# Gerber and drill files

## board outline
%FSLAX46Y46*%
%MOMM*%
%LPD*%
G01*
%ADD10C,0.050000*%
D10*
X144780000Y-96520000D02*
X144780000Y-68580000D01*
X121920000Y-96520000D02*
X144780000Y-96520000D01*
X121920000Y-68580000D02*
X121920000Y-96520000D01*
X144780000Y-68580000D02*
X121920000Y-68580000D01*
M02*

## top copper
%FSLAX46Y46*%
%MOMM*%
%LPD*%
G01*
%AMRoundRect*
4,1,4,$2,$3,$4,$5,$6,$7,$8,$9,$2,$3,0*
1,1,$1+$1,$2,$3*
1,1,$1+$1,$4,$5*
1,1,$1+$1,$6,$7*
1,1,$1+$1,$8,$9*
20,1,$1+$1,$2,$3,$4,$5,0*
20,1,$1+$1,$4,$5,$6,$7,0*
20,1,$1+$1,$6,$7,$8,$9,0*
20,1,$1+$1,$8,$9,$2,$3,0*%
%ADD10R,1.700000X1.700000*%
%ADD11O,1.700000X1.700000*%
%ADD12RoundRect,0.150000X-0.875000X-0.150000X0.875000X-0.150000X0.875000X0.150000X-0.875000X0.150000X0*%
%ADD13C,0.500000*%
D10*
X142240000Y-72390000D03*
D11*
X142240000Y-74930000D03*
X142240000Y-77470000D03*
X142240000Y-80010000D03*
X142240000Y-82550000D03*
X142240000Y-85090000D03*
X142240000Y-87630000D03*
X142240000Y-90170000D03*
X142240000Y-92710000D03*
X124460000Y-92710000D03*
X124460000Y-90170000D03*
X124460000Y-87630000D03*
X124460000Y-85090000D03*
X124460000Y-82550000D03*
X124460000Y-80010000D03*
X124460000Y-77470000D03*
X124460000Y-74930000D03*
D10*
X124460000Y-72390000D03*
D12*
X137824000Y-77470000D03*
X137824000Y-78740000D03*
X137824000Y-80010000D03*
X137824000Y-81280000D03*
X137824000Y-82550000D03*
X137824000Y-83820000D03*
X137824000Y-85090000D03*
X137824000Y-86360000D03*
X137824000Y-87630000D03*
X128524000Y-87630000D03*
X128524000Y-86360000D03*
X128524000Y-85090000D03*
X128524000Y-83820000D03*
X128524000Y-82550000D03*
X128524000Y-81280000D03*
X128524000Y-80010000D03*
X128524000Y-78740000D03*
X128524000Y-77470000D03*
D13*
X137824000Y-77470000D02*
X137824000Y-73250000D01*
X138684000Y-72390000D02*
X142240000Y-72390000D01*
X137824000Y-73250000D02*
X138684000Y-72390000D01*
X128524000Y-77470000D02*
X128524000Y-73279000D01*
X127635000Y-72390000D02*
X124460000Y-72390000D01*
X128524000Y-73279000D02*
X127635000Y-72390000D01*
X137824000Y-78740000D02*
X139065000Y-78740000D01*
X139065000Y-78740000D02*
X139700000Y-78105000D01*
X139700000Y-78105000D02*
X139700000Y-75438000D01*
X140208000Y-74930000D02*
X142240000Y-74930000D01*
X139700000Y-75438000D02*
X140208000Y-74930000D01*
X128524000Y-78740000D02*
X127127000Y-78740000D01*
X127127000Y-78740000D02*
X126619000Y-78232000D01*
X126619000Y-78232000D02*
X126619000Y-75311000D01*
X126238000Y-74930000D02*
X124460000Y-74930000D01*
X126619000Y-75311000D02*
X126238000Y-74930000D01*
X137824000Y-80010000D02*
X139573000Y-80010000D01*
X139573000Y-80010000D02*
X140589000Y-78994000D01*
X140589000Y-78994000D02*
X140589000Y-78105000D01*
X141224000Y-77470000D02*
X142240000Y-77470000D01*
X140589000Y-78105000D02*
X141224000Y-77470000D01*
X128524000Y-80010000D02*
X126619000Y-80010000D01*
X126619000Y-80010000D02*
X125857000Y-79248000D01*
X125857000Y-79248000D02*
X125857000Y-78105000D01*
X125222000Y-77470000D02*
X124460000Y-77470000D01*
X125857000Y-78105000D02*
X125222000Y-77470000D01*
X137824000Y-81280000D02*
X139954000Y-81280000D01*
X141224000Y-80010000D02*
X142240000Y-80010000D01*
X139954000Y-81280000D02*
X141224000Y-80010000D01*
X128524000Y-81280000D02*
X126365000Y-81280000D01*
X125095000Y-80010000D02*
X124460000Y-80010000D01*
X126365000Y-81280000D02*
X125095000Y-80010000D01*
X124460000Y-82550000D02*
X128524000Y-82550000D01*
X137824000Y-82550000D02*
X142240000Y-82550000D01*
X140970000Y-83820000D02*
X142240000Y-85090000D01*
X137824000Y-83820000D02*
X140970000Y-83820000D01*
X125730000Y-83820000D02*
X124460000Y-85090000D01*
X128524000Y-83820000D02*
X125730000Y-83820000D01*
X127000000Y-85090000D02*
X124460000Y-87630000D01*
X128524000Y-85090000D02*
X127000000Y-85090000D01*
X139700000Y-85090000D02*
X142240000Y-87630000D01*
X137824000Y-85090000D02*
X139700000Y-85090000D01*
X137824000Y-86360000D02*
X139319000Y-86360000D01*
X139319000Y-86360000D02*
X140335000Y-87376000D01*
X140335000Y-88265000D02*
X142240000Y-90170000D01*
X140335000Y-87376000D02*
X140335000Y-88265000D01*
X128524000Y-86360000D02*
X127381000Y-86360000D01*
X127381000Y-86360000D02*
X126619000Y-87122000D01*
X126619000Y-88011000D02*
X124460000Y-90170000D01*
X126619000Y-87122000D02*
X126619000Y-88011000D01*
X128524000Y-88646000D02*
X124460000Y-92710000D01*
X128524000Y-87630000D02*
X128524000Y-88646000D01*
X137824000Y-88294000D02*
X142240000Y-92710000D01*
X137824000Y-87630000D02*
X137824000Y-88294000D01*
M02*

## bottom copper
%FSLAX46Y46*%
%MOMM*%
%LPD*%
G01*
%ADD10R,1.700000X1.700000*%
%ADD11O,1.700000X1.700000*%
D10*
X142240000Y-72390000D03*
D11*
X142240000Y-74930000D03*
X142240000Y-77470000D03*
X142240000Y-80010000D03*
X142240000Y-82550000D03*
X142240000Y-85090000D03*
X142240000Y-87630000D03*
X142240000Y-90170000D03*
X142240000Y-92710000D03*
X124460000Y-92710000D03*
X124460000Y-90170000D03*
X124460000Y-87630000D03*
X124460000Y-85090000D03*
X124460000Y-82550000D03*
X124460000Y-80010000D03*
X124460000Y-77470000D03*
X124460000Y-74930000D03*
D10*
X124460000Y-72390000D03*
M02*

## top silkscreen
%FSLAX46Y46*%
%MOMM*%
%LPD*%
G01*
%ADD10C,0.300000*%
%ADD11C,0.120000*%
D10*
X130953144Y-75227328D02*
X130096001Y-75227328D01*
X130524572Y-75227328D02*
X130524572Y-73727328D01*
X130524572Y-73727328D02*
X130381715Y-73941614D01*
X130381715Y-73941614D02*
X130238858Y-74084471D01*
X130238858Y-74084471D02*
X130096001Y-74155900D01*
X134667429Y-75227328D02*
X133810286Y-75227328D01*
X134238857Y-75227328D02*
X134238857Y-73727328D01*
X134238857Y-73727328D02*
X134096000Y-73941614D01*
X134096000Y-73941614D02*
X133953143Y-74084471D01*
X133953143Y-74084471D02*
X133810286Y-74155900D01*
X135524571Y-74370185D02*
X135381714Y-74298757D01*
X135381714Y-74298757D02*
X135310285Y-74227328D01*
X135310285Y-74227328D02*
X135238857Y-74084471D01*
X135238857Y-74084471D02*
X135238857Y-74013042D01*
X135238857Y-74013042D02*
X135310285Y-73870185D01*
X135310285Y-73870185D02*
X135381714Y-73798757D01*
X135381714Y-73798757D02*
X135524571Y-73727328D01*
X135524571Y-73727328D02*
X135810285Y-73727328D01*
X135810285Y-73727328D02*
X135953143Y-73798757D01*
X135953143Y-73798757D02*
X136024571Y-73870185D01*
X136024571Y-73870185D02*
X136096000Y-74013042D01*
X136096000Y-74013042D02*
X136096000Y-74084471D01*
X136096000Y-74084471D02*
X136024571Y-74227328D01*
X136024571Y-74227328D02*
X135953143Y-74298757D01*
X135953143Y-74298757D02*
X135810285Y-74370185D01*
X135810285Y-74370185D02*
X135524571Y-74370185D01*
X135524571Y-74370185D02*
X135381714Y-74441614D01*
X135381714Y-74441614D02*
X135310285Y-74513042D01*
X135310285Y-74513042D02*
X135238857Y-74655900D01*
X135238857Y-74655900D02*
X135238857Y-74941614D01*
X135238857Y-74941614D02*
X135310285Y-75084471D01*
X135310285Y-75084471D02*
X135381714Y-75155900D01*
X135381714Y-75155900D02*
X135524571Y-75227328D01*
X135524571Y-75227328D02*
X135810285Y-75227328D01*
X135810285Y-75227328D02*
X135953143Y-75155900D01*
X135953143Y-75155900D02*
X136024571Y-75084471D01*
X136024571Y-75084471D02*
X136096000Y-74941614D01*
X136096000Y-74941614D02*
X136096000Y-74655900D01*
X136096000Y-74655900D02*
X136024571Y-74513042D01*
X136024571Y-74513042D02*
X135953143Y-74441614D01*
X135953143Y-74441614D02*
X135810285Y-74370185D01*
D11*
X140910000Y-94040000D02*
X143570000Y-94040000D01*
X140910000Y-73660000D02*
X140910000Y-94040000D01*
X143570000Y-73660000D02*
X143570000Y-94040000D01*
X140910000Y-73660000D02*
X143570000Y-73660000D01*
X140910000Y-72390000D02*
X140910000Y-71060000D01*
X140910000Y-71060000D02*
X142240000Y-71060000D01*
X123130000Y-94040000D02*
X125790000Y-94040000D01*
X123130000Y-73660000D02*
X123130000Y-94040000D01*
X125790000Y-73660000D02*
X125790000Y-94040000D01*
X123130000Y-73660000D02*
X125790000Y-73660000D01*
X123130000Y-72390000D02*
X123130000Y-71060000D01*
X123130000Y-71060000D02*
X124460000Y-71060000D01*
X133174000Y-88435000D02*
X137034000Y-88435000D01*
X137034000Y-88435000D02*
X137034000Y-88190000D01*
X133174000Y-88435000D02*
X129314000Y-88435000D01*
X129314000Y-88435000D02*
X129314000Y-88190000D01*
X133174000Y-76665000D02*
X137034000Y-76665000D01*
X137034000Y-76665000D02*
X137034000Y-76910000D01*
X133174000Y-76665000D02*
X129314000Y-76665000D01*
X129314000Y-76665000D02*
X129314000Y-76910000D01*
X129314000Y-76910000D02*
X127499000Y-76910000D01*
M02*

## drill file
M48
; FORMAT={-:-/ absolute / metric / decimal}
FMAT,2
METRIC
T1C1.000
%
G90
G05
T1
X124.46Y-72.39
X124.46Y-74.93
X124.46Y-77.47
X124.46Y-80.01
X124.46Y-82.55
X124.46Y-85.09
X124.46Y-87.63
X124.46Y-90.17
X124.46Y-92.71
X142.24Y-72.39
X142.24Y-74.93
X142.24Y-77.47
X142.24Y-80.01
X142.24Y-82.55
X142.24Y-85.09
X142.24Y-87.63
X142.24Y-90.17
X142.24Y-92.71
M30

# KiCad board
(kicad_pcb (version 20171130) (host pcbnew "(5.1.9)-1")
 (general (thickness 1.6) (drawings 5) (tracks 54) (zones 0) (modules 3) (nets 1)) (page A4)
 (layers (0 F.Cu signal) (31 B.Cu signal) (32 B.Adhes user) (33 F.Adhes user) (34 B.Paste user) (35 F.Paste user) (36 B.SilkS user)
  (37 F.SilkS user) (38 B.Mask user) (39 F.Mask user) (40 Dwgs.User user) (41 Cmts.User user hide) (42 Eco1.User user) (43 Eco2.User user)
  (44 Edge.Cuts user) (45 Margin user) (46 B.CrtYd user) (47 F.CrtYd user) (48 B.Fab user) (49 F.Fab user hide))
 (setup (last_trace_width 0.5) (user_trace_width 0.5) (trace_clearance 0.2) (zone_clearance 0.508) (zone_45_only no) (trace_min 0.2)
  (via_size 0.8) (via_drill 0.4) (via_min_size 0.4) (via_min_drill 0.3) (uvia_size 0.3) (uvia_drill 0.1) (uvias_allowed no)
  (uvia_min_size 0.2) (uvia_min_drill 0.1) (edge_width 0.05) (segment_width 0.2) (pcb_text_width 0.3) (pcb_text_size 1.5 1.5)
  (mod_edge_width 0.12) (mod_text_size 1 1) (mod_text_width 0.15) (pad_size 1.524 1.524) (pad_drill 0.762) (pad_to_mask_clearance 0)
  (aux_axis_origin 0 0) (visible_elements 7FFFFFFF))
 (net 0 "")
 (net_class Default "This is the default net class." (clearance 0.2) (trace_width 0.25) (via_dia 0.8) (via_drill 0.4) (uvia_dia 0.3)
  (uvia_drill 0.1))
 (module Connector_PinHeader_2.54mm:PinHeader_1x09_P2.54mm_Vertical (layer F.Cu) (at 142.24 72.39)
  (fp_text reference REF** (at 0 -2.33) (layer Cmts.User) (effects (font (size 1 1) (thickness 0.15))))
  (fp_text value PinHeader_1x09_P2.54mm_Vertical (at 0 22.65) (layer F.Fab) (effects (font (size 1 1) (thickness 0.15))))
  (fp_line (start -1.33 21.65) (end 1.33 21.65) (layer F.SilkS) (width 0.12))
  (fp_line (start -1.33 1.27) (end -1.33 21.65) (layer F.SilkS) (width 0.12))
  (fp_line (start 1.33 1.27) (end 1.33 21.65) (layer F.SilkS) (width 0.12))
  (fp_line (start -1.33 1.27) (end 1.33 1.27) (layer F.SilkS) (width 0.12))
  (fp_line (start -1.33 0) (end -1.33 -1.33) (layer F.SilkS) (width 0.12))
  (fp_line (start -1.33 -1.33) (end 0 -1.33) (layer F.SilkS) (width 0.12))
  (pad 1 thru_hole rect (at 0 0) (size 1.7 1.7) (drill 1) (layers *.Cu *.Mask))
  (pad 2 thru_hole oval (at 0 2.54) (size 1.7 1.7) (drill 1) (layers *.Cu *.Mask))
  (pad 3 thru_hole oval (at 0 5.08) (size 1.7 1.7) (drill 1) (layers *.Cu *.Mask))
  (pad 4 thru_hole oval (at 0 7.62) (size 1.7 1.7) (drill 1) (layers *.Cu *.Mask))
  (pad 5 thru_hole oval (at 0 10.16) (size 1.7 1.7) (drill 1) (layers *.Cu *.Mask))
  (pad 6 thru_hole oval (at 0 12.7) (size 1.7 1.7) (drill 1) (layers *.Cu *.Mask))
  (pad 7 thru_hole oval (at 0 15.24) (size 1.7 1.7) (drill 1) (layers *.Cu *.Mask))
  (pad 8 thru_hole oval (at 0 17.78) (size 1.7 1.7) (drill 1) (layers *.Cu *.Mask))
  (pad 9 thru_hole oval (at 0 20.32) (size 1.7 1.7) (drill 1) (layers *.Cu *.Mask)))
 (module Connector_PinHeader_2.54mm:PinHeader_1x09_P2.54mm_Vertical (layer F.Cu) (at 124.46 72.39)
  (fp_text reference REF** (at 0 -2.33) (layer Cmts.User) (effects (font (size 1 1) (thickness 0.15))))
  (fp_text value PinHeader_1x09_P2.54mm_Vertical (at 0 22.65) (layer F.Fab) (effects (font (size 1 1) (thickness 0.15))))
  (fp_line (start -1.33 21.65) (end 1.33 21.65) (layer F.SilkS) (width 0.12))
  (fp_line (start -1.33 1.27) (end -1.33 21.65) (layer F.SilkS) (width 0.12))
  (fp_line (start 1.33 1.27) (end 1.33 21.65) (layer F.SilkS) (width 0.12))
  (fp_line (start -1.33 1.27) (end 1.33 1.27) (layer F.SilkS) (width 0.12))
  (fp_line (start -1.33 0) (end -1.33 -1.33) (layer F.SilkS) (width 0.12))
  (fp_line (start -1.33 -1.33) (end 0 -1.33) (layer F.SilkS) (width 0.12))
  (pad 9 thru_hole oval (at 0 20.32) (size 1.7 1.7) (drill 1) (layers *.Cu *.Mask))
  (pad 8 thru_hole oval (at 0 17.78) (size 1.7 1.7) (drill 1) (layers *.Cu *.Mask))
  (pad 7 thru_hole oval (at 0 15.24) (size 1.7 1.7) (drill 1) (layers *.Cu *.Mask))
  (pad 6 thru_hole oval (at 0 12.7) (size 1.7 1.7) (drill 1) (layers *.Cu *.Mask))
  (pad 5 thru_hole oval (at 0 10.16) (size 1.7 1.7) (drill 1) (layers *.Cu *.Mask))
  (pad 4 thru_hole oval (at 0 7.62) (size 1.7 1.7) (drill 1) (layers *.Cu *.Mask))
  (pad 3 thru_hole oval (at 0 5.08) (size 1.7 1.7) (drill 1) (layers *.Cu *.Mask))
  (pad 2 thru_hole oval (at 0 2.54) (size 1.7 1.7) (drill 1) (layers *.Cu *.Mask))
  (pad 1 thru_hole rect (at 0 0) (size 1.7 1.7) (drill 1) (layers *.Cu *.Mask)))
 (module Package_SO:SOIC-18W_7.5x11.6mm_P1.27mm (layer F.Cu) (at 133.174 82.55)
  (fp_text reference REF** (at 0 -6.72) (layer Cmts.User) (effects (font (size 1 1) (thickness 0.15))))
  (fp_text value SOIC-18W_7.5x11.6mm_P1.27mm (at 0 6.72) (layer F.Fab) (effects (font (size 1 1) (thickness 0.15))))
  (fp_line (start 0 5.885) (end 3.86 5.885) (layer F.SilkS) (width 0.12))
  (fp_line (start 3.86 5.885) (end 3.86 5.64) (layer F.SilkS) (width 0.12))
  (fp_line (start 0 5.885) (end -3.86 5.885) (layer F.SilkS) (width 0.12))
  (fp_line (start -3.86 5.885) (end -3.86 5.64) (layer F.SilkS) (width 0.12))
  (fp_line (start 0 -5.885) (end 3.86 -5.885) (layer F.SilkS) (width 0.12))
  (fp_line (start 3.86 -5.885) (end 3.86 -5.64) (layer F.SilkS) (width 0.12))
  (fp_line (start 0 -5.885) (end -3.86 -5.885) (layer F.SilkS) (width 0.12))
  (fp_line (start -3.86 -5.885) (end -3.86 -5.64) (layer F.SilkS) (width 0.12))
  (fp_line (start -3.86 -5.64) (end -5.675 -5.64) (layer F.SilkS) (width 0.12))
  (pad 18 smd roundrect (at 4.65 -5.08) (size 2.05 0.6) (layers F.Cu F.Paste F.Mask) (roundrect_rratio 0.25))
  (pad 17 smd roundrect (at 4.65 -3.81) (size 2.05 0.6) (layers F.Cu F.Paste F.Mask) (roundrect_rratio 0.25))
  (pad 16 smd roundrect (at 4.65 -2.54) (size 2.05 0.6) (layers F.Cu F.Paste F.Mask) (roundrect_rratio 0.25))
  (pad 15 smd roundrect (at 4.65 -1.27) (size 2.05 0.6) (layers F.Cu F.Paste F.Mask) (roundrect_rratio 0.25))
  (pad 14 smd roundrect (at 4.65 0) (size 2.05 0.6) (layers F.Cu F.Paste F.Mask) (roundrect_rratio 0.25))
  (pad 13 smd roundrect (at 4.65 1.27) (size 2.05 0.6) (layers F.Cu F.Paste F.Mask) (roundrect_rratio 0.25))
  (pad 12 smd roundrect (at 4.65 2.54) (size 2.05 0.6) (layers F.Cu F.Paste F.Mask) (roundrect_rratio 0.25))
  (pad 11 smd roundrect (at 4.65 3.81) (size 2.05 0.6) (layers F.Cu F.Paste F.Mask) (roundrect_rratio 0.25))
  (pad 10 smd roundrect (at 4.65 5.08) (size 2.05 0.6) (layers F.Cu F.Paste F.Mask) (roundrect_rratio 0.25))
  (pad 9 smd roundrect (at -4.65 5.08) (size 2.05 0.6) (layers F.Cu F.Paste F.Mask) (roundrect_rratio 0.25))
  (pad 8 smd roundrect (at -4.65 3.81) (size 2.05 0.6) (layers F.Cu F.Paste F.Mask) (roundrect_rratio 0.25))
  (pad 7 smd roundrect (at -4.65 2.54) (size 2.05 0.6) (layers F.Cu F.Paste F.Mask) (roundrect_rratio 0.25))
  (pad 6 smd roundrect (at -4.65 1.27) (size 2.05 0.6) (layers F.Cu F.Paste F.Mask) (roundrect_rratio 0.25))
  (pad 5 smd roundrect (at -4.65 0) (size 2.05 0.6) (layers F.Cu F.Paste F.Mask) (roundrect_rratio 0.25))
  (pad 4 smd roundrect (at -4.65 -1.27) (size 2.05 0.6) (layers F.Cu F.Paste F.Mask) (roundrect_rratio 0.25))
  (pad 3 smd roundrect (at -4.65 -2.54) (size 2.05 0.6) (layers F.Cu F.Paste F.Mask) (roundrect_rratio 0.25))
  (pad 2 smd roundrect (at -4.65 -3.81) (size 2.05 0.6) (layers F.Cu F.Paste F.Mask) (roundrect_rratio 0.25))
  (pad 1 smd roundrect (at -4.65 -5.08) (size 2.05 0.6) (layers F.Cu F.Paste F.Mask) (roundrect_rratio 0.25)))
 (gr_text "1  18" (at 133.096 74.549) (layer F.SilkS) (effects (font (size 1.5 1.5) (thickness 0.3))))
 (gr_line (start 144.78 96.52) (end 144.78 68.58) (layer Edge.Cuts) (width 0.05))
 (gr_line (start 121.92 96.52) (end 144.78 96.52) (layer Edge.Cuts) (width 0.05))
 (gr_line (start 121.92 68.58) (end 121.92 96.52) (layer Edge.Cuts) (width 0.05))
 (gr_line (start 144.78 68.58) (end 121.92 68.58) (layer Edge.Cuts) (width 0.05))
 (segment (start 137.824 77.47) (end 137.824 73.25) (width 0.5) (layer F.Cu) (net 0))
 (segment (start 138.684 72.39) (end 142.24 72.39) (width 0.5) (layer F.Cu) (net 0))
 (segment (start 137.824 73.25) (end 138.684 72.39) (width 0.5) (layer F.Cu) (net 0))
 (segment (start 128.524 77.47) (end 128.524 73.279) (width 0.5) (layer F.Cu) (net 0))
 (segment (start 127.635 72.39) (end 124.46 72.39) (width 0.5) (layer F.Cu) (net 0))
 (segment (start 128.524 73.279) (end 127.635 72.39) (width 0.5) (layer F.Cu) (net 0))
 (segment (start 137.824 78.74) (end 139.065 78.74) (width 0.5) (layer F.Cu) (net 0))
 (segment (start 139.065 78.74) (end 139.7 78.105) (width 0.5) (layer F.Cu) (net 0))
 (segment (start 139.7 78.105) (end 139.7 75.438) (width 0.5) (layer F.Cu) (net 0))
 (segment (start 140.208 74.93) (end 142.24 74.93) (width 0.5) (layer F.Cu) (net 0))
 (segment (start 139.7 75.438) (end 140.208 74.93) (width 0.5) (layer F.Cu) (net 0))
 (segment (start 128.524 78.74) (end 127.127 78.74) (width 0.5) (layer F.Cu) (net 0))
 (segment (start 127.127 78.74) (end 126.619 78.232) (width 0.5) (layer F.Cu) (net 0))
 (segment (start 126.619 78.232) (end 126.619 75.311) (width 0.5) (layer F.Cu) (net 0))
 (segment (start 126.238 74.93) (end 124.46 74.93) (width 0.5) (layer F.Cu) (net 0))
 (segment (start 126.619 75.311) (end 126.238 74.93) (width 0.5) (layer F.Cu) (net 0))
 (segment (start 137.824 80.01) (end 139.573 80.01) (width 0.5) (layer F.Cu) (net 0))
 (segment (start 139.573 80.01) (end 140.589 78.994) (width 0.5) (layer F.Cu) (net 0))
 (segment (start 140.589 78.994) (end 140.589 78.105) (width 0.5) (layer F.Cu) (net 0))
 (segment (start 141.224 77.47) (end 142.24 77.47) (width 0.5) (layer F.Cu) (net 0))
 (segment (start 140.589 78.105) (end 141.224 77.47) (width 0.5) (layer F.Cu) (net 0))
 (segment (start 128.524 80.01) (end 126.619 80.01) (width 0.5) (layer F.Cu) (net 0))
 (segment (start 126.619 80.01) (end 125.857 79.248) (width 0.5) (layer F.Cu) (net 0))
 (segment (start 125.857 79.248) (end 125.857 78.105) (width 0.5) (layer F.Cu) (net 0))
 (segment (start 125.222 77.47) (end 124.46 77.47) (width 0.5) (layer F.Cu) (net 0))
 (segment (start 125.857 78.105) (end 125.222 77.47) (width 0.5) (layer F.Cu) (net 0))
 (segment (start 137.824 81.28) (end 139.954 81.28) (width 0.5) (layer F.Cu) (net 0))
 (segment (start 141.224 80.01) (end 142.24 80.01) (width 0.5) (layer F.Cu) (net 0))
 (segment (start 139.954 81.28) (end 141.224 80.01) (width 0.5) (layer F.Cu) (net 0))
 (segment (start 128.524 81.28) (end 126.365 81.28) (width 0.5) (layer F.Cu) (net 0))
 (segment (start 125.095 80.01) (end 124.46 80.01) (width 0.5) (layer F.Cu) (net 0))
 (segment (start 126.365 81.28) (end 125.095 80.01) (width 0.5) (layer F.Cu) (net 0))
 (segment (start 124.46 82.55) (end 128.524 82.55) (width 0.5) (layer F.Cu) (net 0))
 (segment (start 137.824 82.55) (end 142.24 82.55) (width 0.5) (layer F.Cu) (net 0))
 (segment (start 140.97 83.82) (end 142.24 85.09) (width 0.5) (layer F.Cu) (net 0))
 (segment (start 137.824 83.82) (end 140.97 83.82) (width 0.5) (layer F.Cu) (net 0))
 (segment (start 125.73 83.82) (end 124.46 85.09) (width 0.5) (layer F.Cu) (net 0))
 (segment (start 128.524 83.82) (end 125.73 83.82) (width 0.5) (layer F.Cu) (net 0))
 (segment (start 127 85.09) (end 124.46 87.63) (width 0.5) (layer F.Cu) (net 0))
 (segment (start 128.524 85.09) (end 127 85.09) (width 0.5) (layer F.Cu) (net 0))
 (segment (start 139.7 85.09) (end 142.24 87.63) (width 0.5) (layer F.Cu) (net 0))
 (segment (start 137.824 85.09) (end 139.7 85.09) (width 0.5) (layer F.Cu) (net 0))
 (segment (start 137.824 86.36) (end 139.319 86.36) (width 0.5) (layer F.Cu) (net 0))
 (segment (start 139.319 86.36) (end 140.335 87.376) (width 0.5) (layer F.Cu) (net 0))
 (segment (start 140.335 88.265) (end 142.24 90.17) (width 0.5) (layer F.Cu) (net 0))
 (segment (start 140.335 87.376) (end 140.335 88.265) (width 0.5) (layer F.Cu) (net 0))
 (segment (start 128.524 86.36) (end 127.381 86.36) (width 0.5) (layer F.Cu) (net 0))
 (segment (start 127.381 86.36) (end 126.619 87.122) (width 0.5) (layer F.Cu) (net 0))
 (segment (start 126.619 88.011) (end 124.46 90.17) (width 0.5) (layer F.Cu) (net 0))
 (segment (start 126.619 87.122) (end 126.619 88.011) (width 0.5) (layer F.Cu) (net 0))
 (segment (start 128.524 88.646) (end 124.46 92.71) (width 0.5) (layer F.Cu) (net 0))
 (segment (start 128.524 87.63) (end 128.524 88.646) (width 0.5) (layer F.Cu) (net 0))
 (segment (start 137.824 88.294) (end 142.24 92.71) (width 0.5) (layer F.Cu) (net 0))
 (segment (start 137.824 87.63) (end 137.824 88.294) (width 0.5) (layer F.Cu) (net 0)))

